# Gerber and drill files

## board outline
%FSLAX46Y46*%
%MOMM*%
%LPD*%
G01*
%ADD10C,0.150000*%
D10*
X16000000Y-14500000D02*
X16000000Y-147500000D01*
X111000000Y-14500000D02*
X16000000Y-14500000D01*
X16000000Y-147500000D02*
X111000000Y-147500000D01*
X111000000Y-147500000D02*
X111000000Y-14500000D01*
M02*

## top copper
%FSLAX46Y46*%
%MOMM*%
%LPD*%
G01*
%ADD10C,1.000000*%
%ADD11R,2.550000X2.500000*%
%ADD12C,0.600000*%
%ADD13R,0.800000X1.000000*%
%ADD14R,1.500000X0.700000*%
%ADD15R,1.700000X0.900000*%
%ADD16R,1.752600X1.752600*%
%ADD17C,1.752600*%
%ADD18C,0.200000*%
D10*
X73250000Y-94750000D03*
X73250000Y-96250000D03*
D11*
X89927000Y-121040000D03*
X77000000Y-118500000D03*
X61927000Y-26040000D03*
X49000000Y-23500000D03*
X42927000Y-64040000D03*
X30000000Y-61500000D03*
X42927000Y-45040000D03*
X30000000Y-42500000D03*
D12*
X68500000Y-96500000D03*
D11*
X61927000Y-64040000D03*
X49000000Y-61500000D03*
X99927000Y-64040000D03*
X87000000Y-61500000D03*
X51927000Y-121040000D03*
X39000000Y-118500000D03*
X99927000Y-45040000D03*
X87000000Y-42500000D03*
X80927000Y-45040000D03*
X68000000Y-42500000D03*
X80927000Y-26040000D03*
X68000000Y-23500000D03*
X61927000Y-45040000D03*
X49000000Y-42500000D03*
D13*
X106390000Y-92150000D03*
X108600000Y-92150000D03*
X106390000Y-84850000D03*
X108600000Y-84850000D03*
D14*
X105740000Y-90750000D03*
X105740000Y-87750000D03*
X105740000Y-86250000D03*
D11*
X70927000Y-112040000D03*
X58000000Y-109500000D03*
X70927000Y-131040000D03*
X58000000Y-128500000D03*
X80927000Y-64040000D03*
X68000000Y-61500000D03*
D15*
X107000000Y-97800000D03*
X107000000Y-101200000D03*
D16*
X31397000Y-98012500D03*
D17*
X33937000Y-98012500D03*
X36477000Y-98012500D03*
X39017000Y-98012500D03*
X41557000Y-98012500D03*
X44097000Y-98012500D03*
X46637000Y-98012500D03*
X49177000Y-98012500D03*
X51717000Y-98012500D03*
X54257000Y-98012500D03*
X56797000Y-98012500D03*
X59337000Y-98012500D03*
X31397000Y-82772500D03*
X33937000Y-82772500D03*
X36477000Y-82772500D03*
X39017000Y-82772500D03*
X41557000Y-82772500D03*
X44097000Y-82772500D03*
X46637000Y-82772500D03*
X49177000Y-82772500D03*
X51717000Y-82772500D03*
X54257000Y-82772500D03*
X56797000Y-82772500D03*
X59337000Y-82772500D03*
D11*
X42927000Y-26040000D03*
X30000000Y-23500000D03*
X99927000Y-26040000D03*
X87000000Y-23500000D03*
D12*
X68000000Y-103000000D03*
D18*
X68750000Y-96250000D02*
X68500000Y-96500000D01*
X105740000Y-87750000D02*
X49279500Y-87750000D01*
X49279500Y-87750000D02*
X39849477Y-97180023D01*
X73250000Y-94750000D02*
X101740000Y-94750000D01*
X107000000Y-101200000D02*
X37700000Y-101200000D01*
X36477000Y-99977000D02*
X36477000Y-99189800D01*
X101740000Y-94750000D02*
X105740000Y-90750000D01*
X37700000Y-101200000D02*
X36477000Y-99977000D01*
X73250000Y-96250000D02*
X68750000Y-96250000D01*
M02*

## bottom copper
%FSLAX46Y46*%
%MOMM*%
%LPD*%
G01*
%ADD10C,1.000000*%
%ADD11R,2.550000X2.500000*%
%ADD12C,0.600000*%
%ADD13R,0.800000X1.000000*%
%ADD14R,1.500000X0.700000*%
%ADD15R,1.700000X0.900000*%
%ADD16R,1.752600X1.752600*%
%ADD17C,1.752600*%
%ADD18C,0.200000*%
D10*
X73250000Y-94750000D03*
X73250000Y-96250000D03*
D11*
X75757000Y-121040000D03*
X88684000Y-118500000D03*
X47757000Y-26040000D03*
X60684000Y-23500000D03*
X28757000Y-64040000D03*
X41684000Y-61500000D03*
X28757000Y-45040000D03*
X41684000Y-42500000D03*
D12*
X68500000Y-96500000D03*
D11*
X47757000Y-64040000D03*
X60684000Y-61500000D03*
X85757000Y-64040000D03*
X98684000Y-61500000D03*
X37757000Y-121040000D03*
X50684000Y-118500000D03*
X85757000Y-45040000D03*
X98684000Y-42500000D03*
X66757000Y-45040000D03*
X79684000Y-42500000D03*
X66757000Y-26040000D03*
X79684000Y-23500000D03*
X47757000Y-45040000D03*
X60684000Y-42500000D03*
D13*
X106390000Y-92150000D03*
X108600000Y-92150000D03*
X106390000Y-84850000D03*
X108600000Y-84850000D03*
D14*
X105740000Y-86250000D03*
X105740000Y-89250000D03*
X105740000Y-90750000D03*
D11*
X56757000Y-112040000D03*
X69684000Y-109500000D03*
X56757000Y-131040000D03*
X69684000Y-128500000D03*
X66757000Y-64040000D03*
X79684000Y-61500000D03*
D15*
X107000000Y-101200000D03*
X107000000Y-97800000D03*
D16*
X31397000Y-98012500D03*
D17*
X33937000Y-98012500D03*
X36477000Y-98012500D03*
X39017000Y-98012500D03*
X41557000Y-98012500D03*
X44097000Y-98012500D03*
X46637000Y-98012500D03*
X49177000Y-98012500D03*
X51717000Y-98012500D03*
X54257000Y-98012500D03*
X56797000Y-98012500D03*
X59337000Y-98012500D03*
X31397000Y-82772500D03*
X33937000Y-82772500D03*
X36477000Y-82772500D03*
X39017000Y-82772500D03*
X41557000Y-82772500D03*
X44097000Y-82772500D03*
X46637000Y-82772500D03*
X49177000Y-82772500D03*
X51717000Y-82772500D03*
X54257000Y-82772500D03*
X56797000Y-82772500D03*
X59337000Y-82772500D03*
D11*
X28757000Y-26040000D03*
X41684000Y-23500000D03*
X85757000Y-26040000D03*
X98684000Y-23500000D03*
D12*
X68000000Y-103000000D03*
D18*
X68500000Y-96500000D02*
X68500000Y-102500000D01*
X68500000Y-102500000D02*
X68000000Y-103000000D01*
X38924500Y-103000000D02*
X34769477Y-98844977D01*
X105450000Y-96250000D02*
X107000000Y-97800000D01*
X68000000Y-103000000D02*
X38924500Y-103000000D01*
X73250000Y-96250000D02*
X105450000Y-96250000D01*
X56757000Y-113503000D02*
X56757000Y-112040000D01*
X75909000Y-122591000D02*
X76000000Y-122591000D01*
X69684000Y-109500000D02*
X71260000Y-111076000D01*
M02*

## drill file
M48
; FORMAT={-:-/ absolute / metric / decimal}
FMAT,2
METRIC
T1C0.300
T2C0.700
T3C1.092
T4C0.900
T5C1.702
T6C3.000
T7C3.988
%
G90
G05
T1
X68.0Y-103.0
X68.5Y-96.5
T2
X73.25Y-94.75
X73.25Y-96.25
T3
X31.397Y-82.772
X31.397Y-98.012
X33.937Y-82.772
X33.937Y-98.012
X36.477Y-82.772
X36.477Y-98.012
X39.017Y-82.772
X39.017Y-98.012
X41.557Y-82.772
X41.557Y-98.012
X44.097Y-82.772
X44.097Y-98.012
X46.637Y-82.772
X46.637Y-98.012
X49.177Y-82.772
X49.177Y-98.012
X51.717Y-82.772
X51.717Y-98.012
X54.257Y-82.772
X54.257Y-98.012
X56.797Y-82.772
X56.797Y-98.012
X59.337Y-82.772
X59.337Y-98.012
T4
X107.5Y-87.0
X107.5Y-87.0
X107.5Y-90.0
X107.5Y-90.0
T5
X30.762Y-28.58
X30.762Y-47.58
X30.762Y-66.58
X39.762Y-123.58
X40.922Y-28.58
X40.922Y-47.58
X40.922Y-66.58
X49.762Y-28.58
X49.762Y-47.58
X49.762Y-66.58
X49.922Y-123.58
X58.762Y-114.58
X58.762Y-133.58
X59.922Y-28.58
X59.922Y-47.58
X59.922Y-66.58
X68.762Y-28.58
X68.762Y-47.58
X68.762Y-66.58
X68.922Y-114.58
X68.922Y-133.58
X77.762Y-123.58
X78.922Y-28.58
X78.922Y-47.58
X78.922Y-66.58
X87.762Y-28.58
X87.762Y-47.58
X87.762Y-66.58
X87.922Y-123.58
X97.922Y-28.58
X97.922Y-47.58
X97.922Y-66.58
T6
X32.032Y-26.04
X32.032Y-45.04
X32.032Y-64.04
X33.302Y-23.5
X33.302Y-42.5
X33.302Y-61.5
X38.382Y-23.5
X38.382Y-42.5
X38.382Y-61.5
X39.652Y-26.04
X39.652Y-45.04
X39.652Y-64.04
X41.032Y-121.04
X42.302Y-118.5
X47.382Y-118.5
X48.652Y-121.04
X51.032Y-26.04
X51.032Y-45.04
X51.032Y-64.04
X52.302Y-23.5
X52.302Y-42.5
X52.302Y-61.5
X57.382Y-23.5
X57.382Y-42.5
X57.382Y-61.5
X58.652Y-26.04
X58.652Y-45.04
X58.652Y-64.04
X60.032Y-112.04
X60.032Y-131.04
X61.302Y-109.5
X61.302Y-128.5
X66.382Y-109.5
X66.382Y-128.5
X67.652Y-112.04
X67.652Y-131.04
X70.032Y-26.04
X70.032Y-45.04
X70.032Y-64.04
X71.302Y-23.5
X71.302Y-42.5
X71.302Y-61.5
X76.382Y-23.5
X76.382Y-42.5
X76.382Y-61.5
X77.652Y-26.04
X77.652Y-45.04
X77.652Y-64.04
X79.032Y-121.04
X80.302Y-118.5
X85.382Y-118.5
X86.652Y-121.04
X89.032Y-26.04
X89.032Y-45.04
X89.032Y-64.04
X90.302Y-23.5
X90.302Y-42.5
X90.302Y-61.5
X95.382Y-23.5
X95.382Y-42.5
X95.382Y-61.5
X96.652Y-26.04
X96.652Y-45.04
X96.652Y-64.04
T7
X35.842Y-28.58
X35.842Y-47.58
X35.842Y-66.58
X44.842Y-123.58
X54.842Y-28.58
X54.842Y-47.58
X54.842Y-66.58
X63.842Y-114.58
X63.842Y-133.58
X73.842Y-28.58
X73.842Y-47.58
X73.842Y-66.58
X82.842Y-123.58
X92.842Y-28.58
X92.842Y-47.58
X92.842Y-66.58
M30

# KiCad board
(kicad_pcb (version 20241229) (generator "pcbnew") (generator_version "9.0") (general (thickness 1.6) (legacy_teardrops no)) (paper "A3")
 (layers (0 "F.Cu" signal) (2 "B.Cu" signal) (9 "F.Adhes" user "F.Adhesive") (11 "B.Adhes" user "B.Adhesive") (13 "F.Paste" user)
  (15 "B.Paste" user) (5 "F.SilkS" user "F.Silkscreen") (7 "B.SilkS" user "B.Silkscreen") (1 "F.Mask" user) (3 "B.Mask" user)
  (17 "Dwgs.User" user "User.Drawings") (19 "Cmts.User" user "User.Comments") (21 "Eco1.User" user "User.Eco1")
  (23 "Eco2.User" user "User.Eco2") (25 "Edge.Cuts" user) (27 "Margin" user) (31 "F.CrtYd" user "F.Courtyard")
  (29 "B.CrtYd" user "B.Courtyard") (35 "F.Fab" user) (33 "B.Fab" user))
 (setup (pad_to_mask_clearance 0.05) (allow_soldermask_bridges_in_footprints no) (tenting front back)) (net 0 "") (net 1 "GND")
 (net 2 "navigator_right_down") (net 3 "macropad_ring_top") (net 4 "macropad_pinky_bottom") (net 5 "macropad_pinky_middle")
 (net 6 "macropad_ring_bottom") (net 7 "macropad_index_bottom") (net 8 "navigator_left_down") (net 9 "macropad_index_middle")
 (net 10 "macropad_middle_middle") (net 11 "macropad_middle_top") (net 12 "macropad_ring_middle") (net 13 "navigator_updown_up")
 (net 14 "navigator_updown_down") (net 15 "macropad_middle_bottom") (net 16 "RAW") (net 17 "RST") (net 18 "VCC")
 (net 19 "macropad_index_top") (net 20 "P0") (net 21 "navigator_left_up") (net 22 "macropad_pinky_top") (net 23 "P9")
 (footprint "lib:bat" (layer "F.Cu") (at 73.25 95.5)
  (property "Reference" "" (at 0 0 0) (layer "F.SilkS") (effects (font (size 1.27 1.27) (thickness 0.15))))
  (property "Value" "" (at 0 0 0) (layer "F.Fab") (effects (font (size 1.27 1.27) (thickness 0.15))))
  (pad "1" thru_hole circle (at 0 -0.75 270) (size 1 1) (drill 0.7) (layers "*.Cu" "*.SilkS" "*.Mask") (remove_unused_layers no))
  (pad "2" thru_hole circle (at 0 0.75 270) (size 1 1) (drill 0.7) (layers "*.Cu" "*.SilkS" "*.Mask") (remove_unused_layers no)))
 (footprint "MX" (layer "F.Cu") (at 82.842 123.58)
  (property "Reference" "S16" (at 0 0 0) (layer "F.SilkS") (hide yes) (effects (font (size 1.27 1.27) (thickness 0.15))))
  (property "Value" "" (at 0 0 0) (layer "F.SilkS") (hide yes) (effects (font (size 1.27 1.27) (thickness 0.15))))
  (pad "" np_thru_hole circle (at -5.08 0) (size 1.7018 1.7018) (drill 1.7018) (layers "*.Cu" "*.Mask"))
  (pad "" np_thru_hole circle (at -3.81 -2.54) (size 3 3) (drill 3) (layers "*.Cu" "*.Mask"))
  (pad "" np_thru_hole circle (at -2.54 -5.08) (size 3 3) (drill 3) (layers "*.Cu" "*.Mask"))
  (pad "" np_thru_hole circle (at 0 0) (size 3.9878 3.9878) (drill 3.9878) (layers "*.Cu" "*.Mask"))
  (pad "" np_thru_hole circle (at 2.54 -5.08) (size 3 3) (drill 3) (layers "*.Cu" "*.Mask"))
  (pad "" np_thru_hole circle (at 3.81 -2.54) (size 3 3) (drill 3) (layers "*.Cu" "*.Mask"))
  (pad "" np_thru_hole circle (at 5.08 0) (size 1.7018 1.7018) (drill 1.7018) (layers "*.Cu" "*.Mask"))
  (pad "1" smd rect (at -7.085 -2.54) (size 2.55 2.5) (layers "B.Cu" "B.Mask" "B.Paste") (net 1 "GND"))
  (pad "1" smd rect (at 7.085 -2.54) (size 2.55 2.5) (layers "F.Cu" "F.Mask" "F.Paste") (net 1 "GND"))
  (pad "2" smd rect (at -5.842 -5.08) (size 2.55 2.5) (layers "F.Cu" "F.Mask" "F.Paste") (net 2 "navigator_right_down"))
  (pad "2" smd rect (at 5.842 -5.08) (size 2.55 2.5) (layers "B.Cu" "B.Mask" "B.Paste") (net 2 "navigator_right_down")))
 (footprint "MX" (layer "F.Cu") (at 54.842 28.58)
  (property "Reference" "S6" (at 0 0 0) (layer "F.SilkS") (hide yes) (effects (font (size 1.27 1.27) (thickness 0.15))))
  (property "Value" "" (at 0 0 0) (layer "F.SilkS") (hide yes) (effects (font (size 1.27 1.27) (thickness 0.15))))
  (pad "" np_thru_hole circle (at -5.08 0) (size 1.7018 1.7018) (drill 1.7018) (layers "*.Cu" "*.Mask"))
  (pad "" np_thru_hole circle (at -3.81 -2.54) (size 3 3) (drill 3) (layers "*.Cu" "*.Mask"))
  (pad "" np_thru_hole circle (at -2.54 -5.08) (size 3 3) (drill 3) (layers "*.Cu" "*.Mask"))
  (pad "" np_thru_hole circle (at 0 0) (size 3.9878 3.9878) (drill 3.9878) (layers "*.Cu" "*.Mask"))
  (pad "" np_thru_hole circle (at 2.54 -5.08) (size 3 3) (drill 3) (layers "*.Cu" "*.Mask"))
  (pad "" np_thru_hole circle (at 3.81 -2.54) (size 3 3) (drill 3) (layers "*.Cu" "*.Mask"))
  (pad "" np_thru_hole circle (at 5.08 0) (size 1.7018 1.7018) (drill 1.7018) (layers "*.Cu" "*.Mask"))
  (pad "1" smd rect (at -7.085 -2.54) (size 2.55 2.5) (layers "B.Cu" "B.Mask" "B.Paste") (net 1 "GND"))
  (pad "1" smd rect (at 7.085 -2.54) (size 2.55 2.5) (layers "F.Cu" "F.Mask" "F.Paste") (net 1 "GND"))
  (pad "2" smd rect (at -5.842 -5.08) (size 2.55 2.5) (layers "F.Cu" "F.Mask" "F.Paste") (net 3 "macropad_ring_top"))
  (pad "2" smd rect (at 5.842 -5.08) (size 2.55 2.5) (layers "B.Cu" "B.Mask" "B.Paste") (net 3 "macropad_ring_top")))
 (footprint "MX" (layer "F.Cu") (at 35.842 66.58)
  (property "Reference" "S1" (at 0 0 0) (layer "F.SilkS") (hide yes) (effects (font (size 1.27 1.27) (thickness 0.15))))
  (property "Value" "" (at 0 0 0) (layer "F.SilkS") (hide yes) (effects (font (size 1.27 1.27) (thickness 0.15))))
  (pad "" np_thru_hole circle (at -5.08 0) (size 1.7018 1.7018) (drill 1.7018) (layers "*.Cu" "*.Mask"))
  (pad "" np_thru_hole circle (at -3.81 -2.54) (size 3 3) (drill 3) (layers "*.Cu" "*.Mask"))
  (pad "" np_thru_hole circle (at -2.54 -5.08) (size 3 3) (drill 3) (layers "*.Cu" "*.Mask"))
  (pad "" np_thru_hole circle (at 0 0) (size 3.9878 3.9878) (drill 3.9878) (layers "*.Cu" "*.Mask"))
  (pad "" np_thru_hole circle (at 2.54 -5.08) (size 3 3) (drill 3) (layers "*.Cu" "*.Mask"))
  (pad "" np_thru_hole circle (at 3.81 -2.54) (size 3 3) (drill 3) (layers "*.Cu" "*.Mask"))
  (pad "" np_thru_hole circle (at 5.08 0) (size 1.7018 1.7018) (drill 1.7018) (layers "*.Cu" "*.Mask"))
  (pad "1" smd rect (at -7.085 -2.54) (size 2.55 2.5) (layers "B.Cu" "B.Mask" "B.Paste") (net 1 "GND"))
  (pad "1" smd rect (at 7.085 -2.54) (size 2.55 2.5) (layers "F.Cu" "F.Mask" "F.Paste") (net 1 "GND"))
  (pad "2" smd rect (at -5.842 -5.08) (size 2.55 2.5) (layers "F.Cu" "F.Mask" "F.Paste") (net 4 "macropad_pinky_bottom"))
  (pad "2" smd rect (at 5.842 -5.08) (size 2.55 2.5) (layers "B.Cu" "B.Mask" "B.Paste") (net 4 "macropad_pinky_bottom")))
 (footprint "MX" (layer "F.Cu") (at 35.842 47.58)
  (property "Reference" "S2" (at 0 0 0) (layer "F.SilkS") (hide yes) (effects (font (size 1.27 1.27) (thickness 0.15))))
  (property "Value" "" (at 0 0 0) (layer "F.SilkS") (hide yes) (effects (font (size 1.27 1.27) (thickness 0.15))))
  (pad "" np_thru_hole circle (at -5.08 0) (size 1.7018 1.7018) (drill 1.7018) (layers "*.Cu" "*.Mask"))
  (pad "" np_thru_hole circle (at -3.81 -2.54) (size 3 3) (drill 3) (layers "*.Cu" "*.Mask"))
  (pad "" np_thru_hole circle (at -2.54 -5.08) (size 3 3) (drill 3) (layers "*.Cu" "*.Mask"))
  (pad "" np_thru_hole circle (at 0 0) (size 3.9878 3.9878) (drill 3.9878) (layers "*.Cu" "*.Mask"))
  (pad "" np_thru_hole circle (at 2.54 -5.08) (size 3 3) (drill 3) (layers "*.Cu" "*.Mask"))
  (pad "" np_thru_hole circle (at 3.81 -2.54) (size 3 3) (drill 3) (layers "*.Cu" "*.Mask"))
  (pad "" np_thru_hole circle (at 5.08 0) (size 1.7018 1.7018) (drill 1.7018) (layers "*.Cu" "*.Mask"))
  (pad "1" smd rect (at -7.085 -2.54) (size 2.55 2.5) (layers "B.Cu" "B.Mask" "B.Paste") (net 1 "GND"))
  (pad "1" smd rect (at 7.085 -2.54) (size 2.55 2.5) (layers "F.Cu" "F.Mask" "F.Paste") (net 1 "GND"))
  (pad "2" smd rect (at -5.842 -5.08) (size 2.55 2.5) (layers "F.Cu" "F.Mask" "F.Paste") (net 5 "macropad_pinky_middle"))
  (pad "2" smd rect (at 5.842 -5.08) (size 2.55 2.5) (layers "B.Cu" "B.Mask" "B.Paste") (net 5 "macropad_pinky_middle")))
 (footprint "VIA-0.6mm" (layer "F.Cu") (at 68.5 96.5 110)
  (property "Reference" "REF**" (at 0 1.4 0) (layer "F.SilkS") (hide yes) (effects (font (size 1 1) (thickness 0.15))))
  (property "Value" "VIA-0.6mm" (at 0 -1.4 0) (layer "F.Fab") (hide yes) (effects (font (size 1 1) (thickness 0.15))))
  (pad "1" thru_hole circle (at 0 0) (size 0.6 0.6) (drill 0.3) (layers "*.Cu") (remove_unused_layers no) (zone_connect 2)))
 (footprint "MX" (layer "F.Cu") (at 54.842 66.58)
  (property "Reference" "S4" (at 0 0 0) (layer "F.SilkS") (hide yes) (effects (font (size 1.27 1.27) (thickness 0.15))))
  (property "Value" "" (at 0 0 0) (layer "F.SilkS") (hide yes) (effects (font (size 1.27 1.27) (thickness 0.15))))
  (pad "" np_thru_hole circle (at -5.08 0) (size 1.7018 1.7018) (drill 1.7018) (layers "*.Cu" "*.Mask"))
  (pad "" np_thru_hole circle (at -3.81 -2.54) (size 3 3) (drill 3) (layers "*.Cu" "*.Mask"))
  (pad "" np_thru_hole circle (at -2.54 -5.08) (size 3 3) (drill 3) (layers "*.Cu" "*.Mask"))
  (pad "" np_thru_hole circle (at 0 0) (size 3.9878 3.9878) (drill 3.9878) (layers "*.Cu" "*.Mask"))
  (pad "" np_thru_hole circle (at 2.54 -5.08) (size 3 3) (drill 3) (layers "*.Cu" "*.Mask"))
  (pad "" np_thru_hole circle (at 3.81 -2.54) (size 3 3) (drill 3) (layers "*.Cu" "*.Mask"))
  (pad "" np_thru_hole circle (at 5.08 0) (size 1.7018 1.7018) (drill 1.7018) (layers "*.Cu" "*.Mask"))
  (pad "1" smd rect (at -7.085 -2.54) (size 2.55 2.5) (layers "B.Cu" "B.Mask" "B.Paste") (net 1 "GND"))
  (pad "1" smd rect (at 7.085 -2.54) (size 2.55 2.5) (layers "F.Cu" "F.Mask" "F.Paste") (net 1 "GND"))
  (pad "2" smd rect (at -5.842 -5.08) (size 2.55 2.5) (layers "F.Cu" "F.Mask" "F.Paste") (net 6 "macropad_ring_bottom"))
  (pad "2" smd rect (at 5.842 -5.08) (size 2.55 2.5) (layers "B.Cu" "B.Mask" "B.Paste") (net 6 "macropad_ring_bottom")))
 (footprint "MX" (layer "F.Cu") (at 92.842 66.58)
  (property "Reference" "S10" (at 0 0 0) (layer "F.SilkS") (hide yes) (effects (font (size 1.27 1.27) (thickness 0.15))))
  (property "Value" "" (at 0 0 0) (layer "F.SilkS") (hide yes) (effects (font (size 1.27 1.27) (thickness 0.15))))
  (pad "" np_thru_hole circle (at -5.08 0) (size 1.7018 1.7018) (drill 1.7018) (layers "*.Cu" "*.Mask"))
  (pad "" np_thru_hole circle (at -3.81 -2.54) (size 3 3) (drill 3) (layers "*.Cu" "*.Mask"))
  (pad "" np_thru_hole circle (at -2.54 -5.08) (size 3 3) (drill 3) (layers "*.Cu" "*.Mask"))
  (pad "" np_thru_hole circle (at 0 0) (size 3.9878 3.9878) (drill 3.9878) (layers "*.Cu" "*.Mask"))
  (pad "" np_thru_hole circle (at 2.54 -5.08) (size 3 3) (drill 3) (layers "*.Cu" "*.Mask"))
  (pad "" np_thru_hole circle (at 3.81 -2.54) (size 3 3) (drill 3) (layers "*.Cu" "*.Mask"))
  (pad "" np_thru_hole circle (at 5.08 0) (size 1.7018 1.7018) (drill 1.7018) (layers "*.Cu" "*.Mask"))
  (pad "1" smd rect (at -7.085 -2.54) (size 2.55 2.5) (layers "B.Cu" "B.Mask" "B.Paste") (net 1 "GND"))
  (pad "1" smd rect (at 7.085 -2.54) (size 2.55 2.5) (layers "F.Cu" "F.Mask" "F.Paste") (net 1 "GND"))
  (pad "2" smd rect (at -5.842 -5.08) (size 2.55 2.5) (layers "F.Cu" "F.Mask" "F.Paste") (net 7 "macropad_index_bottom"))
  (pad "2" smd rect (at 5.842 -5.08) (size 2.55 2.5) (layers "B.Cu" "B.Mask" "B.Paste") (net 7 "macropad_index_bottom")))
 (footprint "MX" (layer "F.Cu") (at 44.842 123.58)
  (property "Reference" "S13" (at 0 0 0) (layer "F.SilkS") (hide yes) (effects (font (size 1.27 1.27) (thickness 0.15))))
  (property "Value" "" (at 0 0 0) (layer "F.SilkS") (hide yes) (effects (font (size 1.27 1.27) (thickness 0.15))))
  (pad "" np_thru_hole circle (at -5.08 0) (size 1.7018 1.7018) (drill 1.7018) (layers "*.Cu" "*.Mask"))
  (pad "" np_thru_hole circle (at -3.81 -2.54) (size 3 3) (drill 3) (layers "*.Cu" "*.Mask"))
  (pad "" np_thru_hole circle (at -2.54 -5.08) (size 3 3) (drill 3) (layers "*.Cu" "*.Mask"))
  (pad "" np_thru_hole circle (at 0 0) (size 3.9878 3.9878) (drill 3.9878) (layers "*.Cu" "*.Mask"))
  (pad "" np_thru_hole circle (at 2.54 -5.08) (size 3 3) (drill 3) (layers "*.Cu" "*.Mask"))
  (pad "" np_thru_hole circle (at 3.81 -2.54) (size 3 3) (drill 3) (layers "*.Cu" "*.Mask"))
  (pad "" np_thru_hole circle (at 5.08 0) (size 1.7018 1.7018) (drill 1.7018) (layers "*.Cu" "*.Mask"))
  (pad "1" smd rect (at -7.085 -2.54) (size 2.55 2.5) (layers "B.Cu" "B.Mask" "B.Paste") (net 1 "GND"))
  (pad "1" smd rect (at 7.085 -2.54) (size 2.55 2.5) (layers "F.Cu" "F.Mask" "F.Paste") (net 1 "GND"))
  (pad "2" smd rect (at -5.842 -5.08) (size 2.55 2.5) (layers "F.Cu" "F.Mask" "F.Paste") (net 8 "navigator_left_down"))
  (pad "2" smd rect (at 5.842 -5.08) (size 2.55 2.5) (layers "B.Cu" "B.Mask" "B.Paste") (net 8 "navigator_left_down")))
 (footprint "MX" (layer "F.Cu") (at 92.842 47.58)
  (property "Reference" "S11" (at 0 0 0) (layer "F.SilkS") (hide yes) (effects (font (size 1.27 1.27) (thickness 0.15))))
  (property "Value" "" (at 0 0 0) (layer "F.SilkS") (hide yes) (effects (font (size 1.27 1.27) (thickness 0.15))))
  (pad "" np_thru_hole circle (at -5.08 0) (size 1.7018 1.7018) (drill 1.7018) (layers "*.Cu" "*.Mask"))
  (pad "" np_thru_hole circle (at -3.81 -2.54) (size 3 3) (drill 3) (layers "*.Cu" "*.Mask"))
  (pad "" np_thru_hole circle (at -2.54 -5.08) (size 3 3) (drill 3) (layers "*.Cu" "*.Mask"))
  (pad "" np_thru_hole circle (at 0 0) (size 3.9878 3.9878) (drill 3.9878) (layers "*.Cu" "*.Mask"))
  (pad "" np_thru_hole circle (at 2.54 -5.08) (size 3 3) (drill 3) (layers "*.Cu" "*.Mask"))
  (pad "" np_thru_hole circle (at 3.81 -2.54) (size 3 3) (drill 3) (layers "*.Cu" "*.Mask"))
  (pad "" np_thru_hole circle (at 5.08 0) (size 1.7018 1.7018) (drill 1.7018) (layers "*.Cu" "*.Mask"))
  (pad "1" smd rect (at -7.085 -2.54) (size 2.55 2.5) (layers "B.Cu" "B.Mask" "B.Paste") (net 1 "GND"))
  (pad "1" smd rect (at 7.085 -2.54) (size 2.55 2.5) (layers "F.Cu" "F.Mask" "F.Paste") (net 1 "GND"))
  (pad "2" smd rect (at -5.842 -5.08) (size 2.55 2.5) (layers "F.Cu" "F.Mask" "F.Paste") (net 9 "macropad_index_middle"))
  (pad "2" smd rect (at 5.842 -5.08) (size 2.55 2.5) (layers "B.Cu" "B.Mask" "B.Paste") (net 9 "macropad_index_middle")))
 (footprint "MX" (layer "F.Cu") (at 73.842 47.58)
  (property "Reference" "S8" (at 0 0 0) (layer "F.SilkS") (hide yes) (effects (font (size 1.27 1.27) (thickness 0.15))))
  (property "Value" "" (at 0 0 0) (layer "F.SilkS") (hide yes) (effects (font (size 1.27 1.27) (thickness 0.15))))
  (pad "" np_thru_hole circle (at -5.08 0) (size 1.7018 1.7018) (drill 1.7018) (layers "*.Cu" "*.Mask"))
  (pad "" np_thru_hole circle (at -3.81 -2.54) (size 3 3) (drill 3) (layers "*.Cu" "*.Mask"))
  (pad "" np_thru_hole circle (at -2.54 -5.08) (size 3 3) (drill 3) (layers "*.Cu" "*.Mask"))
  (pad "" np_thru_hole circle (at 0 0) (size 3.9878 3.9878) (drill 3.9878) (layers "*.Cu" "*.Mask"))
  (pad "" np_thru_hole circle (at 2.54 -5.08) (size 3 3) (drill 3) (layers "*.Cu" "*.Mask"))
  (pad "" np_thru_hole circle (at 3.81 -2.54) (size 3 3) (drill 3) (layers "*.Cu" "*.Mask"))
  (pad "" np_thru_hole circle (at 5.08 0) (size 1.7018 1.7018) (drill 1.7018) (layers "*.Cu" "*.Mask"))
  (pad "1" smd rect (at -7.085 -2.54) (size 2.55 2.5) (layers "B.Cu" "B.Mask" "B.Paste") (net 1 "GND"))
  (pad "1" smd rect (at 7.085 -2.54) (size 2.55 2.5) (layers "F.Cu" "F.Mask" "F.Paste") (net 1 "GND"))
  (pad "2" smd rect (at -5.842 -5.08) (size 2.55 2.5) (layers "F.Cu" "F.Mask" "F.Paste") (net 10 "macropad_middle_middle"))
  (pad "2" smd rect (at 5.842 -5.08) (size 2.55 2.5) (layers "B.Cu" "B.Mask" "B.Paste") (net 10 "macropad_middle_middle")))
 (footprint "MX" (layer "F.Cu") (at 73.842 28.58)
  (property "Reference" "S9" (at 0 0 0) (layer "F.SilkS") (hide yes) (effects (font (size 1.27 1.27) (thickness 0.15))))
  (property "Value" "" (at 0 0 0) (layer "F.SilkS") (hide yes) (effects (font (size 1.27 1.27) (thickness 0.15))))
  (pad "" np_thru_hole circle (at -5.08 0) (size 1.7018 1.7018) (drill 1.7018) (layers "*.Cu" "*.Mask"))
  (pad "" np_thru_hole circle (at -3.81 -2.54) (size 3 3) (drill 3) (layers "*.Cu" "*.Mask"))
  (pad "" np_thru_hole circle (at -2.54 -5.08) (size 3 3) (drill 3) (layers "*.Cu" "*.Mask"))
  (pad "" np_thru_hole circle (at 0 0) (size 3.9878 3.9878) (drill 3.9878) (layers "*.Cu" "*.Mask"))
  (pad "" np_thru_hole circle (at 2.54 -5.08) (size 3 3) (drill 3) (layers "*.Cu" "*.Mask"))
  (pad "" np_thru_hole circle (at 3.81 -2.54) (size 3 3) (drill 3) (layers "*.Cu" "*.Mask"))
  (pad "" np_thru_hole circle (at 5.08 0) (size 1.7018 1.7018) (drill 1.7018) (layers "*.Cu" "*.Mask"))
  (pad "1" smd rect (at -7.085 -2.54) (size 2.55 2.5) (layers "B.Cu" "B.Mask" "B.Paste") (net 1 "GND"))
  (pad "1" smd rect (at 7.085 -2.54) (size 2.55 2.5) (layers "F.Cu" "F.Mask" "F.Paste") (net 1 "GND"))
  (pad "2" smd rect (at -5.842 -5.08) (size 2.55 2.5) (layers "F.Cu" "F.Mask" "F.Paste") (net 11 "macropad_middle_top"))
  (pad "2" smd rect (at 5.842 -5.08) (size 2.55 2.5) (layers "B.Cu" "B.Mask" "B.Paste") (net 11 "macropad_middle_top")))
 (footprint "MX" (layer "F.Cu") (at 54.842 47.58)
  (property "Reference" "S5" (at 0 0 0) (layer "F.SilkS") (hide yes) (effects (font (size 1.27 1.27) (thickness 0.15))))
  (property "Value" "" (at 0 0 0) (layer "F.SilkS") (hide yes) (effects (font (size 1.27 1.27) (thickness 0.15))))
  (pad "" np_thru_hole circle (at -5.08 0) (size 1.7018 1.7018) (drill 1.7018) (layers "*.Cu" "*.Mask"))
  (pad "" np_thru_hole circle (at -3.81 -2.54) (size 3 3) (drill 3) (layers "*.Cu" "*.Mask"))
  (pad "" np_thru_hole circle (at -2.54 -5.08) (size 3 3) (drill 3) (layers "*.Cu" "*.Mask"))
  (pad "" np_thru_hole circle (at 0 0) (size 3.9878 3.9878) (drill 3.9878) (layers "*.Cu" "*.Mask"))
  (pad "" np_thru_hole circle (at 2.54 -5.08) (size 3 3) (drill 3) (layers "*.Cu" "*.Mask"))
  (pad "" np_thru_hole circle (at 3.81 -2.54) (size 3 3) (drill 3) (layers "*.Cu" "*.Mask"))
  (pad "" np_thru_hole circle (at 5.08 0) (size 1.7018 1.7018) (drill 1.7018) (layers "*.Cu" "*.Mask"))
  (pad "1" smd rect (at -7.085 -2.54) (size 2.55 2.5) (layers "B.Cu" "B.Mask" "B.Paste") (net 1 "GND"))
  (pad "1" smd rect (at 7.085 -2.54) (size 2.55 2.5) (layers "F.Cu" "F.Mask" "F.Paste") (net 1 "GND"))
  (pad "2" smd rect (at -5.842 -5.08) (size 2.55 2.5) (layers "F.Cu" "F.Mask" "F.Paste") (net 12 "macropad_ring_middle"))
  (pad "2" smd rect (at 5.842 -5.08) (size 2.55 2.5) (layers "B.Cu" "B.Mask" "B.Paste") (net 12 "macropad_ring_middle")))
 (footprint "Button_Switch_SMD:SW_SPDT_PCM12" (layer "F.Cu") (at 107.17 88.5 90)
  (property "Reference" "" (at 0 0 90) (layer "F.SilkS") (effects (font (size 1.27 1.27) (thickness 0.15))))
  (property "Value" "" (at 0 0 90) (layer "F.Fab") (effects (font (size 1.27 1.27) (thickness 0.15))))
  (pad "" smd rect (at -3.65 -0.78 90) (size 1 0.8) (layers "F.Cu" "F.Mask" "F.Paste"))
  (pad "" smd rect (at -3.65 -0.78 90) (size 1 0.8) (layers "B.Cu" "B.Mask" "B.Paste"))
  (pad "" smd rect (at -3.65 1.43 90) (size 1 0.8) (layers "F.Cu" "F.Mask" "F.Paste"))
  (pad "" smd rect (at -3.65 1.43 90) (size 1 0.8) (layers "B.Cu" "B.Mask" "B.Paste"))
  (pad "" np_thru_hole circle (at -1.5 0.33 90) (size 0.9 0.9) (drill 0.9) (layers "*.Cu" "*.Mask"))
  (pad "" np_thru_hole circle (at -1.5 0.33 90) (size 0.9 0.9) (drill 0.9) (layers "*.Cu" "*.Mask"))
  (pad "" np_thru_hole circle (at 1.5 0.33 90) (size 0.9 0.9) (drill 0.9) (layers "*.Cu" "*.Mask"))
  (pad "" np_thru_hole circle (at 1.5 0.33 90) (size 0.9 0.9) (drill 0.9) (layers "*.Cu" "*.Mask"))
  (pad "" smd rect (at 3.65 -0.78 90) (size 1 0.8) (layers "F.Cu" "F.Mask" "F.Paste"))
  (pad "" smd rect (at 3.65 -0.78 90) (size 1 0.8) (layers "B.Cu" "B.Mask" "B.Paste"))
  (pad "" smd rect (at 3.65 1.43 90) (size 1 0.8) (layers "F.Cu" "F.Mask" "F.Paste"))
  (pad "" smd rect (at 3.65 1.43 90) (size 1 0.8) (layers "B.Cu" "B.Mask" "B.Paste"))
  (pad "1" smd rect (at -2.25 -1.43 90) (size 0.7 1.5) (layers "F.Cu" "F.Mask" "F.Paste"))
  (pad "1" smd rect (at 2.25 -1.43 90) (size 0.7 1.5) (layers "B.Cu" "B.Mask" "B.Paste"))
  (pad "2" smd rect (at -0.75 -1.43 90) (size 0.7 1.5) (layers "B.Cu" "B.Mask" "B.Paste"))
  (pad "2" smd rect (at 0.75 -1.43 90) (size 0.7 1.5) (layers "F.Cu" "F.Mask" "F.Paste"))
  (pad "3" smd rect (at -2.25 -1.43 90) (size 0.7 1.5) (layers "B.Cu" "B.Mask" "B.Paste"))
  (pad "3" smd rect (at 2.25 -1.43 90) (size 0.7 1.5) (layers "F.Cu" "F.Mask" "F.Paste")))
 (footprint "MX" (layer "F.Cu") (at 63.842 114.58)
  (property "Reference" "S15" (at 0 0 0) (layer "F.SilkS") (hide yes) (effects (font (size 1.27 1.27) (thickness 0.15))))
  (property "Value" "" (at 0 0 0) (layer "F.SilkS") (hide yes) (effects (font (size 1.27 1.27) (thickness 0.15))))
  (pad "" np_thru_hole circle (at -5.08 0) (size 1.7018 1.7018) (drill 1.7018) (layers "*.Cu" "*.Mask"))
  (pad "" np_thru_hole circle (at -3.81 -2.54) (size 3 3) (drill 3) (layers "*.Cu" "*.Mask"))
  (pad "" np_thru_hole circle (at -2.54 -5.08) (size 3 3) (drill 3) (layers "*.Cu" "*.Mask"))
  (pad "" np_thru_hole circle (at 0 0) (size 3.9878 3.9878) (drill 3.9878) (layers "*.Cu" "*.Mask"))
  (pad "" np_thru_hole circle (at 2.54 -5.08) (size 3 3) (drill 3) (layers "*.Cu" "*.Mask"))
  (pad "" np_thru_hole circle (at 3.81 -2.54) (size 3 3) (drill 3) (layers "*.Cu" "*.Mask"))
  (pad "" np_thru_hole circle (at 5.08 0) (size 1.7018 1.7018) (drill 1.7018) (layers "*.Cu" "*.Mask"))
  (pad "1" smd rect (at -7.085 -2.54) (size 2.55 2.5) (layers "B.Cu" "B.Mask" "B.Paste") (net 1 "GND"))
  (pad "1" smd rect (at 7.085 -2.54) (size 2.55 2.5) (layers "F.Cu" "F.Mask" "F.Paste") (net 1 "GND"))
  (pad "2" smd rect (at -5.842 -5.08) (size 2.55 2.5) (layers "F.Cu" "F.Mask" "F.Paste") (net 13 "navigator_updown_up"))
  (pad "2" smd rect (at 5.842 -5.08) (size 2.55 2.5) (layers "B.Cu" "B.Mask" "B.Paste") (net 13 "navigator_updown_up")))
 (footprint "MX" (layer "F.Cu") (at 63.842 133.58)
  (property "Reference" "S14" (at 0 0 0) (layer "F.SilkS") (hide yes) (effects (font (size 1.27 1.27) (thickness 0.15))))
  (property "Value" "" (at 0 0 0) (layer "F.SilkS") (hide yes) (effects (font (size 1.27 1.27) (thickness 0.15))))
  (pad "" np_thru_hole circle (at -5.08 0) (size 1.7018 1.7018) (drill 1.7018) (layers "*.Cu" "*.Mask"))
  (pad "" np_thru_hole circle (at -3.81 -2.54) (size 3 3) (drill 3) (layers "*.Cu" "*.Mask"))
  (pad "" np_thru_hole circle (at -2.54 -5.08) (size 3 3) (drill 3) (layers "*.Cu" "*.Mask"))
  (pad "" np_thru_hole circle (at 0 0) (size 3.9878 3.9878) (drill 3.9878) (layers "*.Cu" "*.Mask"))
  (pad "" np_thru_hole circle (at 2.54 -5.08) (size 3 3) (drill 3) (layers "*.Cu" "*.Mask"))
  (pad "" np_thru_hole circle (at 3.81 -2.54) (size 3 3) (drill 3) (layers "*.Cu" "*.Mask"))
  (pad "" np_thru_hole circle (at 5.08 0) (size 1.7018 1.7018) (drill 1.7018) (layers "*.Cu" "*.Mask"))
  (pad "1" smd rect (at -7.085 -2.54) (size 2.55 2.5) (layers "B.Cu" "B.Mask" "B.Paste") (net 1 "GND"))
  (pad "1" smd rect (at 7.085 -2.54) (size 2.55 2.5) (layers "F.Cu" "F.Mask" "F.Paste") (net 1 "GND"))
  (pad "2" smd rect (at -5.842 -5.08) (size 2.55 2.5) (layers "F.Cu" "F.Mask" "F.Paste") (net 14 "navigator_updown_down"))
  (pad "2" smd rect (at 5.842 -5.08) (size 2.55 2.5) (layers "B.Cu" "B.Mask" "B.Paste") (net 14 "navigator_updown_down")))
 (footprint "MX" (layer "F.Cu") (at 73.842 66.58)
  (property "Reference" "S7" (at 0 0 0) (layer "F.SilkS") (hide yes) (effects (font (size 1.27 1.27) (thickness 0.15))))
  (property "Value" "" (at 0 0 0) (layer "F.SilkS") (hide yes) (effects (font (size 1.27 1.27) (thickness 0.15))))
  (pad "" np_thru_hole circle (at -5.08 0) (size 1.7018 1.7018) (drill 1.7018) (layers "*.Cu" "*.Mask"))
  (pad "" np_thru_hole circle (at -3.81 -2.54) (size 3 3) (drill 3) (layers "*.Cu" "*.Mask"))
  (pad "" np_thru_hole circle (at -2.54 -5.08) (size 3 3) (drill 3) (layers "*.Cu" "*.Mask"))
  (pad "" np_thru_hole circle (at 0 0) (size 3.9878 3.9878) (drill 3.9878) (layers "*.Cu" "*.Mask"))
  (pad "" np_thru_hole circle (at 2.54 -5.08) (size 3 3) (drill 3) (layers "*.Cu" "*.Mask"))
  (pad "" np_thru_hole circle (at 3.81 -2.54) (size 3 3) (drill 3) (layers "*.Cu" "*.Mask"))
  (pad "" np_thru_hole circle (at 5.08 0) (size 1.7018 1.7018) (drill 1.7018) (layers "*.Cu" "*.Mask"))
  (pad "1" smd rect (at -7.085 -2.54) (size 2.55 2.5) (layers "B.Cu" "B.Mask" "B.Paste") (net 1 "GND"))
  (pad "1" smd rect (at 7.085 -2.54) (size 2.55 2.5) (layers "F.Cu" "F.Mask" "F.Paste") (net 1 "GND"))
  (pad "2" smd rect (at -5.842 -5.08) (size 2.55 2.5) (layers "F.Cu" "F.Mask" "F.Paste") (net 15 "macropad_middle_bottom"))
  (pad "2" smd rect (at 5.842 -5.08) (size 2.55 2.5) (layers "B.Cu" "B.Mask" "B.Paste") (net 15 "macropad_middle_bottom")))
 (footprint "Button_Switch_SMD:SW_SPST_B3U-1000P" (layer "F.Cu") (at 107 99.5 90)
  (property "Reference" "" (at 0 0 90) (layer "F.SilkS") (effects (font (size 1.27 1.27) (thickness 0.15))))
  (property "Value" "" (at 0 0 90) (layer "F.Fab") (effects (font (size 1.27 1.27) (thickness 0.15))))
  (pad "1" smd rect (at -1.7 0 90) (size 0.9 1.7) (layers "B.Cu" "B.Mask" "B.Paste"))
  (pad "1" smd rect (at 1.7 0 90) (size 0.9 1.7) (layers "F.Cu" "F.Mask" "F.Paste"))
  (pad "2" smd rect (at -1.7 0 90) (size 0.9 1.7) (layers "F.Cu" "F.Mask" "F.Paste"))
  (pad "2" smd rect (at 1.7 0 90) (size 0.9 1.7) (layers "B.Cu" "B.Mask" "B.Paste")))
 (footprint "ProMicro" (layer "F.Cu") (at 45.367 90.3925)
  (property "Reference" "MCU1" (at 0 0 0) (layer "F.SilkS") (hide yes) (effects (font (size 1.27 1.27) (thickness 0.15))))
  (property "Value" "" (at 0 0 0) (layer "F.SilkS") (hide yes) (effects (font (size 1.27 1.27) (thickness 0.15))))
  (pad "1" thru_hole rect (at -13.97 7.62) (size 1.7526 1.7526) (drill 1.0922) (layers "*.Cu" "*.SilkS" "*.Mask") (remove_unused_layers no)
   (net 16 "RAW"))
  (pad "2" thru_hole circle (at -11.43 7.62) (size 1.7526 1.7526) (drill 1.0922) (layers "*.Cu" "*.SilkS" "*.Mask")
   (remove_unused_layers no) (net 1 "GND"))
  (pad "3" thru_hole circle (at -8.89 7.62) (size 1.7526 1.7526) (drill 1.0922) (layers "*.Cu" "*.SilkS" "*.Mask") (remove_unused_layers no)
   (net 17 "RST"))
  (pad "4" thru_hole circle (at -6.35 7.62) (size 1.7526 1.7526) (drill 1.0922) (layers "*.Cu" "*.SilkS" "*.Mask") (remove_unused_layers no)
   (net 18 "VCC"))
  (pad "5" thru_hole circle (at -3.81 7.62) (size 1.7526 1.7526) (drill 1.0922) (layers "*.Cu" "*.SilkS" "*.Mask") (remove_unused_layers no)
   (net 5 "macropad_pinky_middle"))
  (pad "6" thru_hole circle (at -1.27 7.62) (size 1.7526 1.7526) (drill 1.0922) (layers "*.Cu" "*.SilkS" "*.Mask") (remove_unused_layers no)
   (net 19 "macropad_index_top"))
  (pad "7" thru_hole circle (at 1.27 7.62) (size 1.7526 1.7526) (drill 1.0922) (layers "*.Cu" "*.SilkS" "*.Mask") (remove_unused_layers no)
   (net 11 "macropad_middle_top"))
  (pad "8" thru_hole circle (at 3.81 7.62) (size 1.7526 1.7526) (drill 1.0922) (layers "*.Cu" "*.SilkS" "*.Mask") (remove_unused_layers no)
   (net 3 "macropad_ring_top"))
  (pad "9" thru_hole circle (at 6.35 7.62) (size 1.7526 1.7526) (drill 1.0922) (layers "*.Cu" "*.SilkS" "*.Mask") (remove_unused_layers no)
   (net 12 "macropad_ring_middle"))
  (pad "10" thru_hole circle (at 8.89 7.62) (size 1.7526 1.7526) (drill 1.0922) (layers "*.Cu" "*.SilkS" "*.Mask") (remove_unused_layers no)
   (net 10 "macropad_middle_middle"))
  (pad "11" thru_hole circle (at 11.43 7.62) (size 1.7526 1.7526) (drill 1.0922) (layers "*.Cu" "*.SilkS" "*.Mask")
   (remove_unused_layers no) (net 9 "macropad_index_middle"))
  (pad "12" thru_hole circle (at 13.97 7.62) (size 1.7526 1.7526) (drill 1.0922) (layers "*.Cu" "*.SilkS" "*.Mask")
   (remove_unused_layers no) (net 4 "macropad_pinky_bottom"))
  (pad "13" thru_hole circle (at -13.97 -7.62) (size 1.7526 1.7526) (drill 1.0922) (layers "*.Cu" "*.SilkS" "*.Mask")
   (remove_unused_layers no) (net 6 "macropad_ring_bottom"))
  (pad "14" thru_hole circle (at -11.43 -7.62) (size 1.7526 1.7526) (drill 1.0922) (layers "*.Cu" "*.SilkS" "*.Mask")
   (remove_unused_layers no) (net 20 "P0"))
  (pad "15" thru_hole circle (at -8.89 -7.62) (size 1.7526 1.7526) (drill 1.0922) (layers "*.Cu" "*.SilkS" "*.Mask")
   (remove_unused_layers no) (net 1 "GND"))
  (pad "16" thru_hole circle (at -6.35 -7.62) (size 1.7526 1.7526) (drill 1.0922) (layers "*.Cu" "*.SilkS" "*.Mask")
   (remove_unused_layers no) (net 1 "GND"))
  (pad "17" thru_hole circle (at -3.81 -7.62) (size 1.7526 1.7526) (drill 1.0922) (layers "*.Cu" "*.SilkS" "*.Mask")
   (remove_unused_layers no) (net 15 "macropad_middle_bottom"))
  (pad "18" thru_hole circle (at -1.27 -7.62) (size 1.7526 1.7526) (drill 1.0922) (layers "*.Cu" "*.SilkS" "*.Mask")
   (remove_unused_layers no) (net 7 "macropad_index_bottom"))
  (pad "19" thru_hole circle (at 1.27 -7.62) (size 1.7526 1.7526) (drill 1.0922) (layers "*.Cu" "*.SilkS" "*.Mask")
   (remove_unused_layers no) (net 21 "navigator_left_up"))
  (pad "20" thru_hole circle (at 3.81 -7.62) (size 1.7526 1.7526) (drill 1.0922) (layers "*.Cu" "*.SilkS" "*.Mask")
   (remove_unused_layers no) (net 13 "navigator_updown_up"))
  (pad "21" thru_hole circle (at 6.35 -7.62) (size 1.7526 1.7526) (drill 1.0922) (layers "*.Cu" "*.SilkS" "*.Mask")
   (remove_unused_layers no) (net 14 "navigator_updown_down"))
  (pad "22" thru_hole circle (at 8.89 -7.62) (size 1.7526 1.7526) (drill 1.0922) (layers "*.Cu" "*.SilkS" "*.Mask")
   (remove_unused_layers no) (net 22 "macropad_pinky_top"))
  (pad "23" thru_hole circle (at 11.43 -7.62) (size 1.7526 1.7526) (drill 1.0922) (layers "*.Cu" "*.SilkS" "*.Mask")
   (remove_unused_layers no) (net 2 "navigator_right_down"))
  (pad "24" thru_hole circle (at 13.97 -7.62) (size 1.7526 1.7526) (drill 1.0922) (layers "*.Cu" "*.SilkS" "*.Mask")
   (remove_unused_layers no) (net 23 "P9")))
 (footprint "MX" (layer "F.Cu") (at 35.842 28.58)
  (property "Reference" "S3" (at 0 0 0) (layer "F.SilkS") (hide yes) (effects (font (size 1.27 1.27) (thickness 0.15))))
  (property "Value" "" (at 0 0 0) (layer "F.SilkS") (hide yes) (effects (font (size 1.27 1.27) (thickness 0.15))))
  (pad "" np_thru_hole circle (at -5.08 0) (size 1.7018 1.7018) (drill 1.7018) (layers "*.Cu" "*.Mask"))
  (pad "" np_thru_hole circle (at -3.81 -2.54) (size 3 3) (drill 3) (layers "*.Cu" "*.Mask"))
  (pad "" np_thru_hole circle (at -2.54 -5.08) (size 3 3) (drill 3) (layers "*.Cu" "*.Mask"))
  (pad "" np_thru_hole circle (at 0 0) (size 3.9878 3.9878) (drill 3.9878) (layers "*.Cu" "*.Mask"))
  (pad "" np_thru_hole circle (at 2.54 -5.08) (size 3 3) (drill 3) (layers "*.Cu" "*.Mask"))
  (pad "" np_thru_hole circle (at 3.81 -2.54) (size 3 3) (drill 3) (layers "*.Cu" "*.Mask"))
  (pad "" np_thru_hole circle (at 5.08 0) (size 1.7018 1.7018) (drill 1.7018) (layers "*.Cu" "*.Mask"))
  (pad "1" smd rect (at -7.085 -2.54) (size 2.55 2.5) (layers "B.Cu" "B.Mask" "B.Paste") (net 1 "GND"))
  (pad "1" smd rect (at 7.085 -2.54) (size 2.55 2.5) (layers "F.Cu" "F.Mask" "F.Paste") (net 1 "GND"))
  (pad "2" smd rect (at -5.842 -5.08) (size 2.55 2.5) (layers "F.Cu" "F.Mask" "F.Paste") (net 22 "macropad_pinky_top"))
  (pad "2" smd rect (at 5.842 -5.08) (size 2.55 2.5) (layers "B.Cu" "B.Mask" "B.Paste") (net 22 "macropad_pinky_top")))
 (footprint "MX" (layer "F.Cu") (at 92.842 28.58)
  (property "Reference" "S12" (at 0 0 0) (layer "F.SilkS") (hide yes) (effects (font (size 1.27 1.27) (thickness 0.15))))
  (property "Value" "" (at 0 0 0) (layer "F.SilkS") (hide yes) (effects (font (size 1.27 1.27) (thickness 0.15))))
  (pad "" np_thru_hole circle (at -5.08 0) (size 1.7018 1.7018) (drill 1.7018) (layers "*.Cu" "*.Mask"))
  (pad "" np_thru_hole circle (at -3.81 -2.54) (size 3 3) (drill 3) (layers "*.Cu" "*.Mask"))
  (pad "" np_thru_hole circle (at -2.54 -5.08) (size 3 3) (drill 3) (layers "*.Cu" "*.Mask"))
  (pad "" np_thru_hole circle (at 0 0) (size 3.9878 3.9878) (drill 3.9878) (layers "*.Cu" "*.Mask"))
  (pad "" np_thru_hole circle (at 2.54 -5.08) (size 3 3) (drill 3) (layers "*.Cu" "*.Mask"))
  (pad "" np_thru_hole circle (at 3.81 -2.54) (size 3 3) (drill 3) (layers "*.Cu" "*.Mask"))
  (pad "" np_thru_hole circle (at 5.08 0) (size 1.7018 1.7018) (drill 1.7018) (layers "*.Cu" "*.Mask"))
  (pad "1" smd rect (at -7.085 -2.54) (size 2.55 2.5) (layers "B.Cu" "B.Mask" "B.Paste") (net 1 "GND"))
  (pad "1" smd rect (at 7.085 -2.54) (size 2.55 2.5) (layers "F.Cu" "F.Mask" "F.Paste") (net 1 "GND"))
  (pad "2" smd rect (at -5.842 -5.08) (size 2.55 2.5) (layers "F.Cu" "F.Mask" "F.Paste") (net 19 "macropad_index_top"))
  (pad "2" smd rect (at 5.842 -5.08) (size 2.55 2.5) (layers "B.Cu" "B.Mask" "B.Paste") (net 19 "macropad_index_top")))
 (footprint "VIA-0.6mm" (layer "F.Cu") (at 68 103 110)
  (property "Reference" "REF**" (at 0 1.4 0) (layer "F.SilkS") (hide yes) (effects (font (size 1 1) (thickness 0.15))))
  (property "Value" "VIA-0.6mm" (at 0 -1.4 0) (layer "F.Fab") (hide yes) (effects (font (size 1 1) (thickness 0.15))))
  (pad "1" thru_hole circle (at 0 0) (size 0.6 0.6) (drill 0.3) (layers "*.Cu") (remove_unused_layers no) (zone_connect 2)))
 (gr_line (start 16 14.5) (end 16 147.5) (stroke (width 0.15) (type solid)) (layer "Edge.Cuts"))
 (gr_line (start 111 14.5) (end 16 14.5) (stroke (width 0.15) (type solid)) (layer "Edge.Cuts"))
 (gr_line (start 16 147.5) (end 111 147.5) (stroke (width 0.15) (type solid)) (layer "Edge.Cuts"))
 (gr_line (start 111 147.5) (end 111 14.5) (stroke (width 0.15) (type solid)) (layer "Edge.Cuts"))
 (segment (start 68.75 96.25) (end 68.5 96.5) (width 0.2) (layer "F.Cu") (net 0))
 (segment (start 105.74 87.75) (end 49.2795 87.75) (width 0.2) (layer "F.Cu") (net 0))
 (segment (start 49.2795 87.75) (end 39.849477 97.180023) (width 0.2) (layer "F.Cu") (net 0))
 (segment (start 73.25 94.75) (end 101.74 94.75) (width 0.2) (layer "F.Cu") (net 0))
 (segment (start 107 101.2) (end 37.7 101.2) (width 0.2) (layer "F.Cu") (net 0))
 (segment (start 36.477 99.977) (end 36.477 99.1898) (width 0.2) (layer "F.Cu") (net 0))
 (segment (start 101.74 94.75) (end 105.74 90.75) (width 0.2) (layer "F.Cu") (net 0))
 (segment (start 37.7 101.2) (end 36.477 99.977) (width 0.2) (layer "F.Cu") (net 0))
 (segment (start 73.25 96.25) (end 68.75 96.25) (width 0.2) (layer "F.Cu") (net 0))
 (segment (start 68.5 96.5) (end 68.5 102.5) (width 0.2) (layer "B.Cu") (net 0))
 (segment (start 68.5 102.5) (end 68 103) (width 0.2) (layer "B.Cu") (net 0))
 (segment (start 38.9245 103) (end 34.769477 98.844977) (width 0.2) (layer "B.Cu") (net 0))
 (segment (start 105.45 96.25) (end 107 97.8) (width 0.2) (layer "B.Cu") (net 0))
 (segment (start 68 103) (end 38.9245 103) (width 0.2) (layer "B.Cu") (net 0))
 (segment (start 73.25 96.25) (end 105.45 96.25) (width 0.2) (layer "B.Cu") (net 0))
 (segment (start 56.757 113.503) (end 56.757 112.04) (width 0.2) (layer "B.Cu") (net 1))
 (segment (start 75.909 122.591) (end 76 122.591) (width 0.2) (layer "B.Cu") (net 13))
 (segment (start 69.684 109.5) (end 71.26 111.076) (width 0.2) (layer "B.Cu") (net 13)))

